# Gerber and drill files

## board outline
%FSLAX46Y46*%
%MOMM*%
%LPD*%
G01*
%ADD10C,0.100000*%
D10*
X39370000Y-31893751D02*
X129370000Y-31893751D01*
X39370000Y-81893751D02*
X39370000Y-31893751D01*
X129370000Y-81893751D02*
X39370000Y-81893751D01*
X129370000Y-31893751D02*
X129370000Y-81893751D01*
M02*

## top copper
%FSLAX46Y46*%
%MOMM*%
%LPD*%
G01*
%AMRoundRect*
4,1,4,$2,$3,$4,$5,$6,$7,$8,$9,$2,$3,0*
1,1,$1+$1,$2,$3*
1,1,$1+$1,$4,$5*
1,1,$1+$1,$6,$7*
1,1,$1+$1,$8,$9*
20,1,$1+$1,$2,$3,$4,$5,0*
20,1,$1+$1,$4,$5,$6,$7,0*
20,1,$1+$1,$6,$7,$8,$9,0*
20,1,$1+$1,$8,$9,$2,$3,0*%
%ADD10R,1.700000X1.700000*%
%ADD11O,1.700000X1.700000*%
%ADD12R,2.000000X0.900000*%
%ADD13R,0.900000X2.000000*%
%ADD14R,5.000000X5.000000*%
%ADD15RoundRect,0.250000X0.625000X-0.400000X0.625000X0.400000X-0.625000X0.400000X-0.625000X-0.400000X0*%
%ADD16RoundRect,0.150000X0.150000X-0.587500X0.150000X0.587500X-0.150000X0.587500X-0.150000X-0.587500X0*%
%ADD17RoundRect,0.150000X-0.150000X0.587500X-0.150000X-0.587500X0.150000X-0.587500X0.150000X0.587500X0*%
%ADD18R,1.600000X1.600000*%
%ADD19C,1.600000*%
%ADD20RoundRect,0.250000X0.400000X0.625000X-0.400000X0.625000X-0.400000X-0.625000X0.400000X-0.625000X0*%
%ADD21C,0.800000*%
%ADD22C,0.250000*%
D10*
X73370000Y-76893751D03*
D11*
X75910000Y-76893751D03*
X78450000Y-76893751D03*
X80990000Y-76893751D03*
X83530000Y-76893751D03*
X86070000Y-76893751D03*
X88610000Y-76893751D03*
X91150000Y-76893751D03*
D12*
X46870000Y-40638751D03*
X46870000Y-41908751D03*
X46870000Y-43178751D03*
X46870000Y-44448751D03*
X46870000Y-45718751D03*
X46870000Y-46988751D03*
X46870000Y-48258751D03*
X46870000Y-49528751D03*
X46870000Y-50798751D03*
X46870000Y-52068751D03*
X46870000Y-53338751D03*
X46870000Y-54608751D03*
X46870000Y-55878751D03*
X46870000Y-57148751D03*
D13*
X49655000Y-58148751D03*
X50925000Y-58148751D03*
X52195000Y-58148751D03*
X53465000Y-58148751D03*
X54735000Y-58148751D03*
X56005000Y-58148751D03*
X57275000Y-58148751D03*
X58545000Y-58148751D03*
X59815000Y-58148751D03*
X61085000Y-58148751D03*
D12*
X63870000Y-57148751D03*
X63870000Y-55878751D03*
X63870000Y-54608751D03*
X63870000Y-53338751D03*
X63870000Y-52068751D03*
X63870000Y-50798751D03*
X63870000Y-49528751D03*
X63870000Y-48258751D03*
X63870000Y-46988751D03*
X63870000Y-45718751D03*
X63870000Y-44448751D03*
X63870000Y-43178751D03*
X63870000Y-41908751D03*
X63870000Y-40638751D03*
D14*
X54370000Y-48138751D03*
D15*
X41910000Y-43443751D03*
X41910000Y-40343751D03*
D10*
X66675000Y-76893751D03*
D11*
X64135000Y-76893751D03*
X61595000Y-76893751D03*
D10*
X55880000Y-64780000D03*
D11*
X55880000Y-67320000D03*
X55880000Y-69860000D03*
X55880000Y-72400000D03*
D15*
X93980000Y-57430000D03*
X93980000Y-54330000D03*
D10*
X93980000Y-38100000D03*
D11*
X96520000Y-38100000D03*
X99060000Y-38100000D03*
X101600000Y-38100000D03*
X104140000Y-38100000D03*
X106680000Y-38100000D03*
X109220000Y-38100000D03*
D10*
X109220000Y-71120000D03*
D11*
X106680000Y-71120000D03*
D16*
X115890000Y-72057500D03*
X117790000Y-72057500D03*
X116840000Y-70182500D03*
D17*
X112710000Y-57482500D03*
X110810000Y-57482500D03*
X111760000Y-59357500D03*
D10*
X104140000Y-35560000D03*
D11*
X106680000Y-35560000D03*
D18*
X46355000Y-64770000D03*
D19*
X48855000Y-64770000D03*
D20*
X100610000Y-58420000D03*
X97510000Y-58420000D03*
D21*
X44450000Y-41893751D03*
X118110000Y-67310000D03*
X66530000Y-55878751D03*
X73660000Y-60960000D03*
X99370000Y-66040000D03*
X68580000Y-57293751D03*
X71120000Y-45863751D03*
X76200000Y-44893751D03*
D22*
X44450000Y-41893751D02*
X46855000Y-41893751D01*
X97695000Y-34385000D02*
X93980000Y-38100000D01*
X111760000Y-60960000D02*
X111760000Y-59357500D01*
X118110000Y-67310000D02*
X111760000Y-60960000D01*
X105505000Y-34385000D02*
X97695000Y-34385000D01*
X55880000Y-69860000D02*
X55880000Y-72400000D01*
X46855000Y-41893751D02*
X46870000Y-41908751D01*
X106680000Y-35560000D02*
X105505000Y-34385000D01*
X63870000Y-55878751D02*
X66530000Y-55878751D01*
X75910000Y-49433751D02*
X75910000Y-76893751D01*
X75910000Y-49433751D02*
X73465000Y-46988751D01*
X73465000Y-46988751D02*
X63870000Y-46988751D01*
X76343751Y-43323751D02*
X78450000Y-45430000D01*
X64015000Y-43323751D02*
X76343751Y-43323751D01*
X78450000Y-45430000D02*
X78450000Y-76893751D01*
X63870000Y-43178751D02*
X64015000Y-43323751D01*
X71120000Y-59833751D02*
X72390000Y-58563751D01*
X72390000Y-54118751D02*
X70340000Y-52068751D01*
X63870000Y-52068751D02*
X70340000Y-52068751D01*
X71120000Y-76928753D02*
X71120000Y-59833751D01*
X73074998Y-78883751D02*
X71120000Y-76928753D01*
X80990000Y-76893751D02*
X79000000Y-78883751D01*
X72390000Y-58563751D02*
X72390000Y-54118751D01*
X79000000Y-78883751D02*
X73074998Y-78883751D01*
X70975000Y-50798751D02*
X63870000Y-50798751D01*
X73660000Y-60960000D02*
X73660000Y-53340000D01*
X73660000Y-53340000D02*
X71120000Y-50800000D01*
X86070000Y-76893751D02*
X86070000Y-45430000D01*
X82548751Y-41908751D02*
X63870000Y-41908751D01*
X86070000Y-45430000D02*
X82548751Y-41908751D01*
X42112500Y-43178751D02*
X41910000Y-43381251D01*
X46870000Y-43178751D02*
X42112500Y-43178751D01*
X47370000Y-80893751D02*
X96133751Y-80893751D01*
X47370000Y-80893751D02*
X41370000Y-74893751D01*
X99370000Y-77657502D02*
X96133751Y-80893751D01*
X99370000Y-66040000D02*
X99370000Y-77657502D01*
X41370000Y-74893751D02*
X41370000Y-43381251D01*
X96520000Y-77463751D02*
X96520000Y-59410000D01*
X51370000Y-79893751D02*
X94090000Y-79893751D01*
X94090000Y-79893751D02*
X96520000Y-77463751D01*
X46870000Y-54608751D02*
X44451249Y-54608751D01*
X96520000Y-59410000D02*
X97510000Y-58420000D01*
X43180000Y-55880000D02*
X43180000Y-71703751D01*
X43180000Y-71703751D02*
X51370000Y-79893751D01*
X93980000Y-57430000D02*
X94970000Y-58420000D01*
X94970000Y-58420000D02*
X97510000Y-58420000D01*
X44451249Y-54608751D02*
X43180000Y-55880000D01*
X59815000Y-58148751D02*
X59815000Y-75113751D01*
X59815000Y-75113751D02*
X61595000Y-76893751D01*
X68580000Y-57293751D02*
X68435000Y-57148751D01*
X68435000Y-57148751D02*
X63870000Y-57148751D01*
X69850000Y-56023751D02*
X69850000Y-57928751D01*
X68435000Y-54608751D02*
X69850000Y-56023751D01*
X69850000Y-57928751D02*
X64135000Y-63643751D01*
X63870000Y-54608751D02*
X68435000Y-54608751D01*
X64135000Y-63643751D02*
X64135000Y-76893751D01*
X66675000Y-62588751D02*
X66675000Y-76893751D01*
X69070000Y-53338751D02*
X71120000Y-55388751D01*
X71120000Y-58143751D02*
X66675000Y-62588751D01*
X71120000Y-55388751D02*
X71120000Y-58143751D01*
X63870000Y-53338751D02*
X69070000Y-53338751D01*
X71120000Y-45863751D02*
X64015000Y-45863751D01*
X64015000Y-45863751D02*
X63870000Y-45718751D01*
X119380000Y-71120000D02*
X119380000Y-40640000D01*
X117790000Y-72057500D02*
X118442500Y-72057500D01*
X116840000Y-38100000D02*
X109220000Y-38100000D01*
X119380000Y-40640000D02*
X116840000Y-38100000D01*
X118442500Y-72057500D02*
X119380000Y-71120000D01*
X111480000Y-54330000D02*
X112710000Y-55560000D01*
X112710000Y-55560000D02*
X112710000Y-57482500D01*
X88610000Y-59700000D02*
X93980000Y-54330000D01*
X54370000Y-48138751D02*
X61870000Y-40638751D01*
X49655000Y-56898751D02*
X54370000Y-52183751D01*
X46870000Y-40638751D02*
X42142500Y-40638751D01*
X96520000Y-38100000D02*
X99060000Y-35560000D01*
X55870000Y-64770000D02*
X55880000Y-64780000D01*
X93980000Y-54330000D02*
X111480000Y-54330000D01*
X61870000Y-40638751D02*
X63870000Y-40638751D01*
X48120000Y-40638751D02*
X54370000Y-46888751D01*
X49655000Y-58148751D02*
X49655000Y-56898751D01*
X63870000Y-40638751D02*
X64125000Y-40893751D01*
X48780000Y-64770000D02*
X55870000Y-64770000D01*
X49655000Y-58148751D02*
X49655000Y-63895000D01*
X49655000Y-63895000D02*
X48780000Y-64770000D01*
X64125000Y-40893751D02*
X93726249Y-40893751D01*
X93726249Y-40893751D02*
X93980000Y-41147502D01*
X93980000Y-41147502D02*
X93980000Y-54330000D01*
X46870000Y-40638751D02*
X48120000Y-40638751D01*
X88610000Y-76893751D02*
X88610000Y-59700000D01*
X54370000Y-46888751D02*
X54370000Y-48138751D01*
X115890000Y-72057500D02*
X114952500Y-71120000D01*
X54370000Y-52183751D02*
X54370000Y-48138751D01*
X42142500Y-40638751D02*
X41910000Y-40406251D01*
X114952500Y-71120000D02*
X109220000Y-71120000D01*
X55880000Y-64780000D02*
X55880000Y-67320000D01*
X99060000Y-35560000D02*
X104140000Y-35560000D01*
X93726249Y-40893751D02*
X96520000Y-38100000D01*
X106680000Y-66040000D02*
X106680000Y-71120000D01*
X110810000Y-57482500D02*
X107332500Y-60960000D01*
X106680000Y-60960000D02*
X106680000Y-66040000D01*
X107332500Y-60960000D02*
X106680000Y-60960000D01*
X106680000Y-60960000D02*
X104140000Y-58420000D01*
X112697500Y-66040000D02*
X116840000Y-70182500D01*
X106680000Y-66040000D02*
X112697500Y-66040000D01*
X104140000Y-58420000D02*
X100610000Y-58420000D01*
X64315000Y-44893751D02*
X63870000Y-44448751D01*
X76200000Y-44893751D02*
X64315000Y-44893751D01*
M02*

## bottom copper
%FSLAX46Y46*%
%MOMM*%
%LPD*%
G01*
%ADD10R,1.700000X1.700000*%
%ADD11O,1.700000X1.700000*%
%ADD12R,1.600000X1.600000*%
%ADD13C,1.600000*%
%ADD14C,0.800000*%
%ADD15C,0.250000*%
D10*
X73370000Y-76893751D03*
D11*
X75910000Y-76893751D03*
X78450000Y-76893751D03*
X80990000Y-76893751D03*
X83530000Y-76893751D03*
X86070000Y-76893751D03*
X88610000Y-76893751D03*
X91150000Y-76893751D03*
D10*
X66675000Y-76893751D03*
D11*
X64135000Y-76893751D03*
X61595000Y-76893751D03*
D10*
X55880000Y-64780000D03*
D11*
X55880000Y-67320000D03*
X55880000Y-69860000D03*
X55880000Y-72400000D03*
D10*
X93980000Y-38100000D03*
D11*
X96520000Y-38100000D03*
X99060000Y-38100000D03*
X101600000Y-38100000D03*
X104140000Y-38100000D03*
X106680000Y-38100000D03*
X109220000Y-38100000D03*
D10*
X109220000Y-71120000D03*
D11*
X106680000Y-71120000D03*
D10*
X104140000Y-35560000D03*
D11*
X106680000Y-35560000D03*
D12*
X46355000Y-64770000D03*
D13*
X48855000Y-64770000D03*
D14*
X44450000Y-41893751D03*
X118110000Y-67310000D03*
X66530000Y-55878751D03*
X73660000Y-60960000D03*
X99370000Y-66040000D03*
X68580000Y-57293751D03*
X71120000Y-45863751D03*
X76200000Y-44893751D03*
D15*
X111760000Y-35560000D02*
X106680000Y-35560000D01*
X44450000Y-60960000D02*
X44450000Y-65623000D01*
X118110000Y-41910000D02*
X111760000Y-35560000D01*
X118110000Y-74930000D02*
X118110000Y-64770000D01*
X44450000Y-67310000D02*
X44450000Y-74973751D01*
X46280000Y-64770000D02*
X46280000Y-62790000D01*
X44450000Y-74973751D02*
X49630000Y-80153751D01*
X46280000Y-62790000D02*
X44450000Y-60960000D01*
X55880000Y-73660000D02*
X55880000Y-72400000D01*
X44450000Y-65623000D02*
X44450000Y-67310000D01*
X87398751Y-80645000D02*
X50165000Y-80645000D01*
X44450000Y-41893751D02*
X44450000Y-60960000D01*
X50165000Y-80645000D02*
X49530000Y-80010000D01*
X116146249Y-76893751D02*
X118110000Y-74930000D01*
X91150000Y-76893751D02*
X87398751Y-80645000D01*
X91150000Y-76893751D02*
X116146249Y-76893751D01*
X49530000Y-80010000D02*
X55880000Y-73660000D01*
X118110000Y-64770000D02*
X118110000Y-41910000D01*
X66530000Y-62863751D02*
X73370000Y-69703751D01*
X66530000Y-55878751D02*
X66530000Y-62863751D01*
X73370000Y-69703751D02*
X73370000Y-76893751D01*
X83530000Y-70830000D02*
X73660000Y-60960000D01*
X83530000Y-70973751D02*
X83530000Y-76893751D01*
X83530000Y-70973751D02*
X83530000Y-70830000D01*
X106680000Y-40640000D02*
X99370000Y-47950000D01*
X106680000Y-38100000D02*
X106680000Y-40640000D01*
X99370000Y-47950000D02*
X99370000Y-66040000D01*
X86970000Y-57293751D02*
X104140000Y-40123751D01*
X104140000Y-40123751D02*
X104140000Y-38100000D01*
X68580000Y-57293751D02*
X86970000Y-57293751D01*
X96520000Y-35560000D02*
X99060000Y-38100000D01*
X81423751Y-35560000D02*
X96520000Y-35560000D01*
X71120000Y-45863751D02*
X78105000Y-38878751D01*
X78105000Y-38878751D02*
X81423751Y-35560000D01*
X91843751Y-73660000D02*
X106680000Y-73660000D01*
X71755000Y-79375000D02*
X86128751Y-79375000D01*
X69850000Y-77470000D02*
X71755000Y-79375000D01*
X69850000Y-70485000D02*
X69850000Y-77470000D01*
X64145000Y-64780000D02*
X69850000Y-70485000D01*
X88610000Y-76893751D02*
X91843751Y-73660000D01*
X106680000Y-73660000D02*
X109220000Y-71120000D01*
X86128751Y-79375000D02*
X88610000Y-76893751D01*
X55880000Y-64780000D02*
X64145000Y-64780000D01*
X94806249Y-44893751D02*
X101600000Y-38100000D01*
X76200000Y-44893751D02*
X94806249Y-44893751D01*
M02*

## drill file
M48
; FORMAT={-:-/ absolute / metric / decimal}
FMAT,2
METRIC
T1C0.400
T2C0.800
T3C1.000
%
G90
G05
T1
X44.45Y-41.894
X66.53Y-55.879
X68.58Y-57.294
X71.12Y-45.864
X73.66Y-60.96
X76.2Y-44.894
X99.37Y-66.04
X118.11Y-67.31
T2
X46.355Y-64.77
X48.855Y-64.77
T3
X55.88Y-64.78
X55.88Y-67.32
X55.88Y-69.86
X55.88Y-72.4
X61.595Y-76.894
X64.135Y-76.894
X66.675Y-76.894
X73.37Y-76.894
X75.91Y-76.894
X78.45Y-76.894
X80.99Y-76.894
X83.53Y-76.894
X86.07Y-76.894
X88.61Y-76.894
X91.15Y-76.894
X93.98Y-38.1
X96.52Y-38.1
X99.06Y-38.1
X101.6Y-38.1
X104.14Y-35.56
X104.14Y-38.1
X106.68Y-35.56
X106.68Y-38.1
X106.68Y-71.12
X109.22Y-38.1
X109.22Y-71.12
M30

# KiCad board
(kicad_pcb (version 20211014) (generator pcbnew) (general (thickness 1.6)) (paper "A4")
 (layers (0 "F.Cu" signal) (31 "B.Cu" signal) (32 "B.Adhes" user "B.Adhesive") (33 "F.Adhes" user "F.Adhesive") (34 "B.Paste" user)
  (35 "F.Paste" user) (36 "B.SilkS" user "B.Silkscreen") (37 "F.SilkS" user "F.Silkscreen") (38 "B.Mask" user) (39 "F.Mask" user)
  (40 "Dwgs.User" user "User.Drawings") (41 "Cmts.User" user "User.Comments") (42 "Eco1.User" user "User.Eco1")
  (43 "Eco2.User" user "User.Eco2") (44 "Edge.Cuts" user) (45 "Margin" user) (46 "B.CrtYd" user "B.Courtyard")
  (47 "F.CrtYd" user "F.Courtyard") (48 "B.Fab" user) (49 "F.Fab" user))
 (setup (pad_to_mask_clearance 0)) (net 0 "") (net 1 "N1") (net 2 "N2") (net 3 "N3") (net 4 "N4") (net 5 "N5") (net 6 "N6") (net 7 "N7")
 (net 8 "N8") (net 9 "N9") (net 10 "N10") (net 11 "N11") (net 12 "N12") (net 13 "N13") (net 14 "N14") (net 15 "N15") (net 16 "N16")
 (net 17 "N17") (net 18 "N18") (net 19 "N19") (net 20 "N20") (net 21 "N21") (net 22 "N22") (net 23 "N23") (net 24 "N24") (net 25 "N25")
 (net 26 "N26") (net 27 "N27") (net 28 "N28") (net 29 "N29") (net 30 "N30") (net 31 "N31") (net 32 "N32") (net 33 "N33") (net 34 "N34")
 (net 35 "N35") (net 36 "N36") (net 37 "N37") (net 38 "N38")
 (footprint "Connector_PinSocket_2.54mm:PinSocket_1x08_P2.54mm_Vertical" (layer "F.Cu") (at 73.37 76.893751 90)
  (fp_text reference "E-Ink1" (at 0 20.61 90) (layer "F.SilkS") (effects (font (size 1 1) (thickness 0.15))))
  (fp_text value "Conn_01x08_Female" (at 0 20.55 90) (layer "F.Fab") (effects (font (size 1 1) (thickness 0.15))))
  (pad "1" thru_hole rect locked (at 0 0 90) (size 1.7 1.7) (drill 1) (layers *.Cu *.Mask) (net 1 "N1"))
  (pad "2" thru_hole oval locked (at 0 2.54 90) (size 1.7 1.7) (drill 1) (layers *.Cu *.Mask) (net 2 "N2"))
  (pad "3" thru_hole oval locked (at 0 5.08 90) (size 1.7 1.7) (drill 1) (layers *.Cu *.Mask) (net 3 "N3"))
  (pad "4" thru_hole oval locked (at 0 7.62 90) (size 1.7 1.7) (drill 1) (layers *.Cu *.Mask) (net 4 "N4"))
  (pad "5" thru_hole oval locked (at 0 10.16 90) (size 1.7 1.7) (drill 1) (layers *.Cu *.Mask) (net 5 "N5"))
  (pad "6" thru_hole oval locked (at 0 12.7 90) (size 1.7 1.7) (drill 1) (layers *.Cu *.Mask) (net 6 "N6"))
  (pad "7" thru_hole oval locked (at 0 15.24 90) (size 1.7 1.7) (drill 1) (layers *.Cu *.Mask) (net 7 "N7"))
  (pad "8" thru_hole oval locked (at 0 17.78 90) (size 1.7 1.7) (drill 1) (layers *.Cu *.Mask) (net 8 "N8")))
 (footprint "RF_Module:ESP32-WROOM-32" (layer "F.Cu") (at 55.37 48.893751)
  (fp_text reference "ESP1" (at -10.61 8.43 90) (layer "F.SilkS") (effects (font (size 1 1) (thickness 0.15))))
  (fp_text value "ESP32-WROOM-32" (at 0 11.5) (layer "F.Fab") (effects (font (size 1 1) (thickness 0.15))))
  (pad "1" smd rect locked (at -8.5 -8.255) (size 2 0.9) (layers "F.Cu" "F.Paste" "F.Mask") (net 7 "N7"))
  (pad "2" smd rect locked (at -8.5 -6.985) (size 2 0.9) (layers "F.Cu" "F.Paste" "F.Mask") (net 8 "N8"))
  (pad "3" smd rect locked (at -8.5 -5.715) (size 2 0.9) (layers "F.Cu" "F.Paste" "F.Mask") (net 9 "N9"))
  (pad "4" smd rect locked (at -8.5 -4.445) (size 2 0.9) (layers "F.Cu" "F.Paste" "F.Mask") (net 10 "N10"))
  (pad "5" smd rect locked (at -8.5 -3.175) (size 2 0.9) (layers "F.Cu" "F.Paste" "F.Mask") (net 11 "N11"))
  (pad "6" smd rect locked (at -8.5 -1.905) (size 2 0.9) (layers "F.Cu" "F.Paste" "F.Mask") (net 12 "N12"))
  (pad "7" smd rect locked (at -8.5 -0.635) (size 2 0.9) (layers "F.Cu" "F.Paste" "F.Mask") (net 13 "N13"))
  (pad "8" smd rect locked (at -8.5 0.635) (size 2 0.9) (layers "F.Cu" "F.Paste" "F.Mask") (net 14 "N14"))
  (pad "9" smd rect locked (at -8.5 1.905) (size 2 0.9) (layers "F.Cu" "F.Paste" "F.Mask") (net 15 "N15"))
  (pad "10" smd rect locked (at -8.5 3.175) (size 2 0.9) (layers "F.Cu" "F.Paste" "F.Mask") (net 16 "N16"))
  (pad "11" smd rect locked (at -8.5 4.445) (size 2 0.9) (layers "F.Cu" "F.Paste" "F.Mask") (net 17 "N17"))
  (pad "12" smd rect locked (at -8.5 5.715) (size 2 0.9) (layers "F.Cu" "F.Paste" "F.Mask") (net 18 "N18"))
  (pad "13" smd rect locked (at -8.5 6.985) (size 2 0.9) (layers "F.Cu" "F.Paste" "F.Mask") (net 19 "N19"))
  (pad "14" smd rect locked (at -8.5 8.255) (size 2 0.9) (layers "F.Cu" "F.Paste" "F.Mask") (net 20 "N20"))
  (pad "15" smd rect locked (at -5.715 9.255 90) (size 2 0.9) (layers "F.Cu" "F.Paste" "F.Mask") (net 7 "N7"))
  (pad "16" smd rect locked (at -4.445 9.255 90) (size 2 0.9) (layers "F.Cu" "F.Paste" "F.Mask") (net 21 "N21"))
  (pad "17" smd rect locked (at -3.175 9.255 90) (size 2 0.9) (layers "F.Cu" "F.Paste" "F.Mask") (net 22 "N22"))
  (pad "18" smd rect locked (at -1.905 9.255 90) (size 2 0.9) (layers "F.Cu" "F.Paste" "F.Mask") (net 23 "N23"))
  (pad "19" smd rect locked (at -0.635 9.255 90) (size 2 0.9) (layers "F.Cu" "F.Paste" "F.Mask") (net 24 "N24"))
  (pad "20" smd rect locked (at 0.635 9.255 90) (size 2 0.9) (layers "F.Cu" "F.Paste" "F.Mask") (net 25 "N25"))
  (pad "21" smd rect locked (at 1.905 9.255 90) (size 2 0.9) (layers "F.Cu" "F.Paste" "F.Mask") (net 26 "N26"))
  (pad "22" smd rect locked (at 3.175 9.255 90) (size 2 0.9) (layers "F.Cu" "F.Paste" "F.Mask") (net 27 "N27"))
  (pad "23" smd rect locked (at 4.445 9.255 90) (size 2 0.9) (layers "F.Cu" "F.Paste" "F.Mask") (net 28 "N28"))
  (pad "24" smd rect locked (at 5.715 9.255 90) (size 2 0.9) (layers "F.Cu" "F.Paste" "F.Mask") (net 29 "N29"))
  (pad "25" smd rect locked (at 8.5 8.255) (size 2 0.9) (layers "F.Cu" "F.Paste" "F.Mask") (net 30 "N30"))
  (pad "26" smd rect locked (at 8.5 6.985) (size 2 0.9) (layers "F.Cu" "F.Paste" "F.Mask") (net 1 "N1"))
  (pad "27" smd rect locked (at 8.5 5.715) (size 2 0.9) (layers "F.Cu" "F.Paste" "F.Mask") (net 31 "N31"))
  (pad "28" smd rect locked (at 8.5 4.445) (size 2 0.9) (layers "F.Cu" "F.Paste" "F.Mask") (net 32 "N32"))
  (pad "29" smd rect locked (at 8.5 3.175) (size 2 0.9) (layers "F.Cu" "F.Paste" "F.Mask") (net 4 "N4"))
  (pad "30" smd rect locked (at 8.5 1.905) (size 2 0.9) (layers "F.Cu" "F.Paste" "F.Mask") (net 5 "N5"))
  (pad "31" smd rect locked (at 8.5 0.635) (size 2 0.9) (layers "F.Cu" "F.Paste" "F.Mask") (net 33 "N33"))
  (pad "32" smd rect locked (at 8.5 -0.635) (size 2 0.9) (layers "F.Cu" "F.Paste" "F.Mask") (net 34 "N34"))
  (pad "33" smd rect locked (at 8.5 -1.905) (size 2 0.9) (layers "F.Cu" "F.Paste" "F.Mask") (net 2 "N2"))
  (pad "34" smd rect locked (at 8.5 -3.175) (size 2 0.9) (layers "F.Cu" "F.Paste" "F.Mask") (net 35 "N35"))
  (pad "35" smd rect locked (at 8.5 -4.445) (size 2 0.9) (layers "F.Cu" "F.Paste" "F.Mask") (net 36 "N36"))
  (pad "36" smd rect locked (at 8.5 -5.715) (size 2 0.9) (layers "F.Cu" "F.Paste" "F.Mask") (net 3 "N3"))
  (pad "37" smd rect locked (at 8.5 -6.985) (size 2 0.9) (layers "F.Cu" "F.Paste" "F.Mask") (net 6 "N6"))
  (pad "38" smd rect locked (at 8.5 -8.255) (size 2 0.9) (layers "F.Cu" "F.Paste" "F.Mask") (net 7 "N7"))
  (pad "39" smd rect locked (at -1 -0.755) (size 5 5) (layers "F.Cu" "F.Paste" "F.Mask") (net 7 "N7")))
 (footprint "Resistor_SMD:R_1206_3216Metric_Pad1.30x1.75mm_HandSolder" (layer "F.Cu") (at 41.91 41.893751 90)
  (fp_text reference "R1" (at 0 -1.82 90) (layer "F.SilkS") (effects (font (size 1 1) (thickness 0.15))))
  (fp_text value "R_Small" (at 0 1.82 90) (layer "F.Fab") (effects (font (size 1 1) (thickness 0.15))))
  (pad "1" smd roundrect (at -1.55 0 90) (size 1.3 1.75) (layers "F.Cu" "F.Paste" "F.Mask") (roundrect_rratio 0.192308) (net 9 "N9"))
  (pad "2" smd roundrect (at 1.55 0 90) (size 1.3 1.75) (layers "F.Cu" "F.Paste" "F.Mask") (roundrect_rratio 0.192308) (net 7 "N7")))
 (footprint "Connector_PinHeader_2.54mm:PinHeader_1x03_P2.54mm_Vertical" (layer "F.Cu") (at 66.675 76.893751 -90)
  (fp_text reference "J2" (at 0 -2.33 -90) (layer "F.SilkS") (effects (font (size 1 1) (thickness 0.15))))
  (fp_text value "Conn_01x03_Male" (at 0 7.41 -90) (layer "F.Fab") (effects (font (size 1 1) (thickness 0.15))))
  (pad "1" thru_hole rect (at 0 0 270) (size 1.7 1.7) (drill 1) (layers *.Cu *.Mask) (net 32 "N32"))
  (pad "2" thru_hole oval (at 0 2.54 270) (size 1.7 1.7) (drill 1) (layers *.Cu *.Mask) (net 31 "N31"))
  (pad "3" thru_hole oval (at 0 5.08 270) (size 1.7 1.7) (drill 1) (layers *.Cu *.Mask) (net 28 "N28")))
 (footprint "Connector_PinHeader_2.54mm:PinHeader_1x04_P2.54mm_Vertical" (layer "F.Cu") (at 55.88 64.78)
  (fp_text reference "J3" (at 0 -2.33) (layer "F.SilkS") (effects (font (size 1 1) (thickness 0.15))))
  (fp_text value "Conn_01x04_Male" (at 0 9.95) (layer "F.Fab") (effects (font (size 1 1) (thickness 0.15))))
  (pad "1" thru_hole rect (at 0 0) (size 1.7 1.7) (drill 1) (layers *.Cu *.Mask) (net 7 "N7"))
  (pad "2" thru_hole oval (at 0 2.54) (size 1.7 1.7) (drill 1) (layers *.Cu *.Mask) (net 7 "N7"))
  (pad "3" thru_hole oval (at 0 5.08) (size 1.7 1.7) (drill 1) (layers *.Cu *.Mask) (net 8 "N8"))
  (pad "4" thru_hole oval (at 0 7.62) (size 1.7 1.7) (drill 1) (layers *.Cu *.Mask) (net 8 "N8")))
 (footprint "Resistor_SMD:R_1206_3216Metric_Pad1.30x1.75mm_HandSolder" (layer "F.Cu") (at 93.98 55.88 90)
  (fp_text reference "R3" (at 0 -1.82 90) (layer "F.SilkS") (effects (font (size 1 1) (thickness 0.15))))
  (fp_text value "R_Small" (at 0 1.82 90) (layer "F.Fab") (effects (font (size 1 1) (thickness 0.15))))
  (pad "1" smd roundrect (at -1.55 0 90) (size 1.3 1.75) (layers "F.Cu" "F.Paste" "F.Mask") (roundrect_rratio 0.192308) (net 18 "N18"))
  (pad "2" smd roundrect (at 1.55 0 90) (size 1.3 1.75) (layers "F.Cu" "F.Paste" "F.Mask") (roundrect_rratio 0.192308) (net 7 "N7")))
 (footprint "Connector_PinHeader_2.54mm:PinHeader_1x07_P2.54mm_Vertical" (layer "F.Cu") (at 93.98 38.1 90)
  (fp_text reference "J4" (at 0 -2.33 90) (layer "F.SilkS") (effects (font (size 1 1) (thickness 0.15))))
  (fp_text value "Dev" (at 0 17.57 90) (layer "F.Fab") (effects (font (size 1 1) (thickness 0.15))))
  (pad "1" thru_hole rect (at 0 0 90) (size 1.7 1.7) (drill 1) (layers *.Cu *.Mask) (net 8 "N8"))
  (pad "2" thru_hole oval (at 0 2.54 90) (size 1.7 1.7) (drill 1) (layers *.Cu *.Mask) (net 7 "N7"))
  (pad "3" thru_hole oval (at 0 5.08 90) (size 1.7 1.7) (drill 1) (layers *.Cu *.Mask) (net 35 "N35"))
  (pad "4" thru_hole oval (at 0 7.62 90) (size 1.7 1.7) (drill 1) (layers *.Cu *.Mask) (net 36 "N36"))
  (pad "5" thru_hole oval (at 0 10.16 90) (size 1.7 1.7) (drill 1) (layers *.Cu *.Mask) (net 30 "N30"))
  (pad "6" thru_hole oval (at 0 12.7 90) (size 1.7 1.7) (drill 1) (layers *.Cu *.Mask) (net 9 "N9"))
  (pad "7" thru_hole oval (at 0 15.24 90) (size 1.7 1.7) (drill 1) (layers *.Cu *.Mask) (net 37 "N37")))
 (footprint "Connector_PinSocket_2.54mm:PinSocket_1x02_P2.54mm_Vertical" (layer "F.Cu") (at 109.22 71.12 -90)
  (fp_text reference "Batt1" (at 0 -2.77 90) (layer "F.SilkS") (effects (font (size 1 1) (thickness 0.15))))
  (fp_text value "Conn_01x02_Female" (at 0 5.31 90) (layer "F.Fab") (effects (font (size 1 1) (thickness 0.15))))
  (pad "1" thru_hole rect (at 0 0 270) (size 1.7 1.7) (drill 1) (layers *.Cu *.Mask) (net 7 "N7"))
  (pad "2" thru_hole oval (at 0 2.54 270) (size 1.7 1.7) (drill 1) (layers *.Cu *.Mask) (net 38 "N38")))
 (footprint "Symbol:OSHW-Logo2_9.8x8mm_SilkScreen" (layer "F.Cu") (at 122.555 38.735)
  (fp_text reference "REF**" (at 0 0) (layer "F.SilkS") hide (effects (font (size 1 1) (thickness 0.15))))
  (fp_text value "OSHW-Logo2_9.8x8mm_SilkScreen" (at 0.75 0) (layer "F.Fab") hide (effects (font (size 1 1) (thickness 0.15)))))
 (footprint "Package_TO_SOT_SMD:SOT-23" (layer "F.Cu") (at 116.84 71.12 90)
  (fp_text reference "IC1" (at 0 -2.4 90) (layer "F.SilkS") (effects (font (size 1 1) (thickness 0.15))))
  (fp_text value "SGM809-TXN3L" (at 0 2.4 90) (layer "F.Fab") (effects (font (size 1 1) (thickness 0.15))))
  (pad "1" smd roundrect (at -0.9375 -0.95 90) (size 1.475 0.6) (layers "F.Cu" "F.Paste" "F.Mask") (roundrect_rratio 0.25) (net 7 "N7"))
  (pad "2" smd roundrect (at -0.9375 0.95 90) (size 1.475 0.6) (layers "F.Cu" "F.Paste" "F.Mask") (roundrect_rratio 0.25) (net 37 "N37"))
  (pad "3" smd roundrect (at 0.9375 0 90) (size 1.475 0.6) (layers "F.Cu" "F.Paste" "F.Mask") (roundrect_rratio 0.25) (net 38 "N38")))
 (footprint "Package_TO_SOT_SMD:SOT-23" (layer "F.Cu") (at 111.76 58.42 -90)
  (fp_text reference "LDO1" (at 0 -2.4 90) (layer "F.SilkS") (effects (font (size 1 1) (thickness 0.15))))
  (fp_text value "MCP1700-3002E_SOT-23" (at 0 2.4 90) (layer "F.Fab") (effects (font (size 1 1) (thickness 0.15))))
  (pad "1" smd roundrect (at -0.9375 -0.95 270) (size 1.475 0.6) (layers "F.Cu" "F.Paste" "F.Mask") (roundrect_rratio 0.25) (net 7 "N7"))
  (pad "2" smd roundrect (at -0.9375 0.95 270) (size 1.475 0.6) (layers "F.Cu" "F.Paste" "F.Mask") (roundrect_rratio 0.25) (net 38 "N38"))
  (pad "3" smd roundrect (at 0.9375 0 270) (size 1.475 0.6) (layers "F.Cu" "F.Paste" "F.Mask") (roundrect_rratio 0.25) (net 8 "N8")))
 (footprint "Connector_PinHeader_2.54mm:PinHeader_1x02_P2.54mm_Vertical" (layer "F.Cu") (at 104.14 35.56 90)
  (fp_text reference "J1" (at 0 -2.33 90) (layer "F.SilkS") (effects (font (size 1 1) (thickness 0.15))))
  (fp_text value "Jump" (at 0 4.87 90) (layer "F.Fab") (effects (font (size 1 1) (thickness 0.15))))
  (pad "1" thru_hole rect (at 0 0 90) (size 1.7 1.7) (drill 1) (layers *.Cu *.Mask) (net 7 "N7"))
  (pad "2" thru_hole oval (at 0 2.54 90) (size 1.7 1.7) (drill 1) (layers *.Cu *.Mask) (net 8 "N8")))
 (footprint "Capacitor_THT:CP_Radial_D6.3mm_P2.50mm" (layer "F.Cu") (at 46.355 64.77)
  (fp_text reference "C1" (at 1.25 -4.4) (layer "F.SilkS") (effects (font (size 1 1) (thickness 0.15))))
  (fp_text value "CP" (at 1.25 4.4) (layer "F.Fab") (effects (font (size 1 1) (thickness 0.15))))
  (pad "1" thru_hole rect (at 0 0) (size 1.6 1.6) (drill 0.8) (layers *.Cu *.Mask) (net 8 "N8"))
  (pad "2" thru_hole circle (at 2.5 0) (size 1.6 1.6) (drill 0.8) (layers *.Cu *.Mask) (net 7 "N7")))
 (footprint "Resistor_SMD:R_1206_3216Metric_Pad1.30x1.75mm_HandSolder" (layer "F.Cu") (at 99.06 58.42 180)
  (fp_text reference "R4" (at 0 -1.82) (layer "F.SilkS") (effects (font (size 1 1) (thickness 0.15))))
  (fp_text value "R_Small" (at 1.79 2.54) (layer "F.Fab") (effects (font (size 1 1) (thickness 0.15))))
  (pad "1" smd roundrect (at -1.55 0 180) (size 1.3 1.75) (layers "F.Cu" "F.Paste" "F.Mask") (roundrect_rratio 0.192308) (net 38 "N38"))
  (pad "2" smd roundrect (at 1.55 0 180) (size 1.3 1.75) (layers "F.Cu" "F.Paste" "F.Mask") (roundrect_rratio 0.192308) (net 18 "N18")))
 (gr_line (start 39.37 31.893751) (end 129.37 31.893751) (layer "Edge.Cuts") (width 0.1))
 (gr_line (start 39.37 81.893751) (end 39.37 31.893751) (layer "Edge.Cuts") (width 0.1))
 (gr_line (start 129.37 81.893751) (end 39.37 81.893751) (layer "Edge.Cuts") (width 0.1))
 (gr_line (start 129.37 31.893751) (end 129.37 81.893751) (layer "Edge.Cuts") (width 0.1))
 (segment (start 44.45 41.893751) (end 46.855 41.893751) (width 0.25) (layer "F.Cu") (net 8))
 (segment (start 97.695 34.385) (end 93.98 38.1) (width 0.25) (layer "F.Cu") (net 8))
 (segment (start 111.76 60.96) (end 111.76 59.3575) (width 0.25) (layer "F.Cu") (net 8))
 (segment (start 118.11 67.31) (end 111.76 60.96) (width 0.25) (layer "F.Cu") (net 8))
 (segment (start 105.505 34.385) (end 97.695 34.385) (width 0.25) (layer "F.Cu") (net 8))
 (segment (start 55.88 69.86) (end 55.88 72.4) (width 0.25) (layer "F.Cu") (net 8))
 (segment (start 46.855 41.893751) (end 46.87 41.908751) (width 0.25) (layer "F.Cu") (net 8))
 (segment (start 106.68 35.56) (end 105.505 34.385) (width 0.25) (layer "F.Cu") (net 8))
 (via (at 44.45 41.893751) (size 0.8) (drill 0.4) (layers "F.Cu" "B.Cu") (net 8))
 (via (at 118.11 67.31) (size 0.8) (drill 0.4) (layers "F.Cu" "B.Cu") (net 8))
 (segment (start 111.76 35.56) (end 106.68 35.56) (width 0.25) (layer "B.Cu") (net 8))
 (segment (start 44.45 60.96) (end 44.45 65.623) (width 0.25) (layer "B.Cu") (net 8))
 (segment (start 118.11 41.91) (end 111.76 35.56) (width 0.25) (layer "B.Cu") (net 8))
 (segment (start 118.11 74.93) (end 118.11 64.77) (width 0.25) (layer "B.Cu") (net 8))
 (segment (start 44.45 67.31) (end 44.45 74.973751) (width 0.25) (layer "B.Cu") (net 8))
 (segment (start 46.28 64.77) (end 46.28 62.79) (width 0.25) (layer "B.Cu") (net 8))
 (segment (start 44.45 74.973751) (end 49.63 80.153751) (width 0.25) (layer "B.Cu") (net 8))
 (segment (start 46.28 62.79) (end 44.45 60.96) (width 0.25) (layer "B.Cu") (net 8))
 (segment (start 55.88 73.66) (end 55.88 72.4) (width 0.25) (layer "B.Cu") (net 8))
 (segment (start 44.45 65.623) (end 44.45 67.31) (width 0.25) (layer "B.Cu") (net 8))
 (segment (start 87.398751 80.645) (end 50.165 80.645) (width 0.25) (layer "B.Cu") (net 8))
 (segment (start 44.45 41.893751) (end 44.45 60.96) (width 0.25) (layer "B.Cu") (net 8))
 (segment (start 50.165 80.645) (end 49.53 80.01) (width 0.25) (layer "B.Cu") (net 8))
 (segment (start 116.146249 76.893751) (end 118.11 74.93) (width 0.25) (layer "B.Cu") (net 8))
 (segment (start 91.15 76.893751) (end 87.398751 80.645) (width 0.25) (layer "B.Cu") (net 8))
 (segment (start 91.15 76.893751) (end 116.146249 76.893751) (width 0.25) (layer "B.Cu") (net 8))
 (segment (start 49.53 80.01) (end 55.88 73.66) (width 0.25) (layer "B.Cu") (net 8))
 (segment (start 118.11 64.77) (end 118.11 41.91) (width 0.25) (layer "B.Cu") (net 8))
 (segment (start 63.87 55.878751) (end 66.53 55.878751) (width 0.25) (layer "F.Cu") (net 1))
 (via (at 66.53 55.878751) (size 0.8) (drill 0.4) (layers "F.Cu" "B.Cu") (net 1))
 (segment (start 66.53 62.863751) (end 73.37 69.703751) (width 0.25) (layer "B.Cu") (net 1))
 (segment (start 66.53 55.878751) (end 66.53 62.863751) (width 0.25) (layer "B.Cu") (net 1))
 (segment (start 73.37 69.703751) (end 73.37 76.893751) (width 0.25) (layer "B.Cu") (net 1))
 (segment (start 75.91 49.433751) (end 75.91 76.893751) (width 0.25) (layer "F.Cu") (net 2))
 (segment (start 75.91 49.433751) (end 73.465 46.988751) (width 0.25) (layer "F.Cu") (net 2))
 (segment (start 73.465 46.988751) (end 63.87 46.988751) (width 0.25) (layer "F.Cu") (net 2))
 (segment (start 76.343751 43.323751) (end 78.45 45.43) (width 0.25) (layer "F.Cu") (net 3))
 (segment (start 64.015 43.323751) (end 76.343751 43.323751) (width 0.25) (layer "F.Cu") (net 3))
 (segment (start 78.45 45.43) (end 78.45 76.893751) (width 0.25) (layer "F.Cu") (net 3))
 (segment (start 63.87 43.178751) (end 64.015 43.323751) (width 0.25) (layer "F.Cu") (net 3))
 (segment (start 71.12 59.833751) (end 72.39 58.563751) (width 0.25) (layer "F.Cu") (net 4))
 (segment (start 72.39 54.118751) (end 70.34 52.068751) (width 0.25) (layer "F.Cu") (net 4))
 (segment (start 63.87 52.068751) (end 70.34 52.068751) (width 0.25) (layer "F.Cu") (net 4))
 (segment (start 71.12 76.928753) (end 71.12 59.833751) (width 0.25) (layer "F.Cu") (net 4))
 (segment (start 73.074998 78.883751) (end 71.12 76.928753) (width 0.25) (layer "F.Cu") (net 4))
 (segment (start 80.99 76.893751) (end 79 78.883751) (width 0.25) (layer "F.Cu") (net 4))
 (segment (start 72.39 58.563751) (end 72.39 54.118751) (width 0.25) (layer "F.Cu") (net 4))
 (segment (start 79 78.883751) (end 73.074998 78.883751) (width 0.25) (layer "F.Cu") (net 4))
 (segment (start 70.975 50.798751) (end 63.87 50.798751) (width 0.25) (layer "F.Cu") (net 5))
 (segment (start 73.66 60.96) (end 73.66 53.34) (width 0.25) (layer "F.Cu") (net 5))
 (segment (start 73.66 53.34) (end 71.12 50.8) (width 0.25) (layer "F.Cu") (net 5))
 (via (at 73.66 60.96) (size 0.8) (drill 0.4) (layers "F.Cu" "B.Cu") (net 5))
 (segment (start 83.53 70.83) (end 73.66 60.96) (width 0.25) (layer "B.Cu") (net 5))
 (segment (start 83.53 70.973751) (end 83.53 76.893751) (width 0.25) (layer "B.Cu") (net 5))
 (segment (start 83.53 70.973751) (end 83.53 70.83) (width 0.25) (layer "B.Cu") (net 5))
 (segment (start 86.07 76.893751) (end 86.07 45.43) (width 0.25) (layer "F.Cu") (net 6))
 (segment (start 82.548751 41.908751) (end 63.87 41.908751) (width 0.25) (layer "F.Cu") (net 6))
 (segment (start 86.07 45.43) (end 82.548751 41.908751) (width 0.25) (layer "F.Cu") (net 6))
 (segment (start 42.1125 43.178751) (end 41.91 43.381251) (width 0.25) (layer "F.Cu") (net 9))
 (segment (start 46.87 43.178751) (end 42.1125 43.178751) (width 0.25) (layer "F.Cu") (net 9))
 (segment (start 47.37 80.893751) (end 96.133751 80.893751) (width 0.25) (layer "F.Cu") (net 9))
 (segment (start 47.37 80.893751) (end 41.37 74.893751) (width 0.25) (layer "F.Cu") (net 9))
 (segment (start 99.37 77.657502) (end 96.133751 80.893751) (width 0.25) (layer "F.Cu") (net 9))
 (segment (start 99.37 66.04) (end 99.37 77.657502) (width 0.25) (layer "F.Cu") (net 9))
 (segment (start 41.37 74.893751) (end 41.37 43.381251) (width 0.25) (layer "F.Cu") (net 9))
 (via (at 99.37 66.04) (size 0.8) (drill 0.4) (layers "F.Cu" "B.Cu") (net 9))
 (segment (start 106.68 40.64) (end 99.37 47.95) (width 0.25) (layer "B.Cu") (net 9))
 (segment (start 106.68 38.1) (end 106.68 40.64) (width 0.25) (layer "B.Cu") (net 9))
 (segment (start 99.37 47.95) (end 99.37 66.04) (width 0.25) (layer "B.Cu") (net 9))
 (segment (start 96.52 77.463751) (end 96.52 59.41) (width 0.25) (layer "F.Cu") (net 18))
 (segment (start 51.37 79.893751) (end 94.09 79.893751) (width 0.25) (layer "F.Cu") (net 18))
 (segment (start 94.09 79.893751) (end 96.52 77.463751) (width 0.25) (layer "F.Cu") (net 18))
 (segment (start 46.87 54.608751) (end 44.451249 54.608751) (width 0.25) (layer "F.Cu") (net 18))
 (segment (start 96.52 59.41) (end 97.51 58.42) (width 0.25) (layer "F.Cu") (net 18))
 (segment (start 43.18 55.88) (end 43.18 71.703751) (width 0.25) (layer "F.Cu") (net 18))
 (segment (start 43.18 71.703751) (end 51.37 79.893751) (width 0.25) (layer "F.Cu") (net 18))
 (segment (start 93.98 57.43) (end 94.97 58.42) (width 0.25) (layer "F.Cu") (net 18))
 (segment (start 94.97 58.42) (end 97.51 58.42) (width 0.25) (layer "F.Cu") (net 18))
 (segment (start 44.451249 54.608751) (end 43.18 55.88) (width 0.25) (layer "F.Cu") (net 18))
 (segment (start 59.815 58.148751) (end 59.815 75.113751) (width 0.25) (layer "F.Cu") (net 28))
 (segment (start 59.815 75.113751) (end 61.595 76.893751) (width 0.25) (layer "F.Cu") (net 28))
 (segment (start 68.58 57.293751) (end 68.435 57.148751) (width 0.25) (layer "F.Cu") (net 30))
 (segment (start 68.435 57.148751) (end 63.87 57.148751) (width 0.25) (layer "F.Cu") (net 30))
 (via (at 68.58 57.293751) (size 0.8) (drill 0.4) (layers "F.Cu" "B.Cu") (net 30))
 (segment (start 86.97 57.293751) (end 104.14 40.123751) (width 0.25) (layer "B.Cu") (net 30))
 (segment (start 104.14 40.123751) (end 104.14 38.1) (width 0.25) (layer "B.Cu") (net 30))
 (segment (start 68.58 57.293751) (end 86.97 57.293751) (width 0.25) (layer "B.Cu") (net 30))
 (segment (start 69.85 56.023751) (end 69.85 57.928751) (width 0.25) (layer "F.Cu") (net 31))
 (segment (start 68.435 54.608751) (end 69.85 56.023751) (width 0.25) (layer "F.Cu") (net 31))
 (segment (start 69.85 57.928751) (end 64.135 63.643751) (width 0.25) (layer "F.Cu") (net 31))
 (segment (start 63.87 54.608751) (end 68.435 54.608751) (width 0.25) (layer "F.Cu") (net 31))
 (segment (start 64.135 63.643751) (end 64.135 76.893751) (width 0.25) (layer "F.Cu") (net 31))
 (segment (start 66.675 62.588751) (end 66.675 76.893751) (width 0.25) (layer "F.Cu") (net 32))
 (segment (start 69.07 53.338751) (end 71.12 55.388751) (width 0.25) (layer "F.Cu") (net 32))
 (segment (start 71.12 58.143751) (end 66.675 62.588751) (width 0.25) (layer "F.Cu") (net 32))
 (segment (start 71.12 55.388751) (end 71.12 58.143751) (width 0.25) (layer "F.Cu") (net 32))
 (segment (start 63.87 53.338751) (end 69.07 53.338751) (width 0.25) (layer "F.Cu") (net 32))
 (segment (start 71.12 45.863751) (end 64.015 45.863751) (width 0.25) (layer "F.Cu") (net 35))
 (segment (start 64.015 45.863751) (end 63.87 45.718751) (width 0.25) (layer "F.Cu") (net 35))
 (via (at 71.12 45.863751) (size 0.8) (drill 0.4) (layers "F.Cu" "B.Cu") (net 35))
 (segment (start 96.52 35.56) (end 99.06 38.1) (width 0.25) (layer "B.Cu") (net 35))
 (segment (start 81.423751 35.56) (end 96.52 35.56) (width 0.25) (layer "B.Cu") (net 35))
 (segment (start 71.12 45.863751) (end 78.105 38.878751) (width 0.25) (layer "B.Cu") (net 35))
 (segment (start 78.105 38.878751) (end 81.423751 35.56) (width 0.25) (layer "B.Cu") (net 35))
 (segment (start 119.38 71.12) (end 119.38 40.64) (width 0.25) (layer "F.Cu") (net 37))
 (segment (start 117.79 72.0575) (end 118.4425 72.0575) (width 0.25) (layer "F.Cu") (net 37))
 (segment (start 116.84 38.1) (end 109.22 38.1) (width 0.25) (layer "F.Cu") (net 37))
 (segment (start 119.38 40.64) (end 116.84 38.1) (width 0.25) (layer "F.Cu") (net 37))
 (segment (start 118.4425 72.0575) (end 119.38 71.12) (width 0.25) (layer "F.Cu") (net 37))
 (segment (start 111.48 54.33) (end 112.71 55.56) (width 0.25) (layer "F.Cu") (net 7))
 (segment (start 112.71 55.56) (end 112.71 57.4825) (width 0.25) (layer "F.Cu") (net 7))
 (segment (start 88.61 59.7) (end 93.98 54.33) (width 0.25) (layer "F.Cu") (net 7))
 (segment (start 54.37 48.138751) (end 61.87 40.638751) (width 0.25) (layer "F.Cu") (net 7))
 (segment (start 49.655 56.898751) (end 54.37 52.183751) (width 0.25) (layer "F.Cu") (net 7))
 (segment (start 46.87 40.638751) (end 42.1425 40.638751) (width 0.25) (layer "F.Cu") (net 7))
 (segment (start 96.52 38.1) (end 99.06 35.56) (width 0.25) (layer "F.Cu") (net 7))
 (segment (start 55.87 64.77) (end 55.88 64.78) (width 0.25) (layer "F.Cu") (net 7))
 (segment (start 93.98 54.33) (end 111.48 54.33) (width 0.25) (layer "F.Cu") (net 7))
 (segment (start 61.87 40.638751) (end 63.87 40.638751) (width 0.25) (layer "F.Cu") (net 7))
 (segment (start 48.12 40.638751) (end 54.37 46.888751) (width 0.25) (layer "F.Cu") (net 7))
 (segment (start 49.655 58.148751) (end 49.655 56.898751) (width 0.25) (layer "F.Cu") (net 7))
 (segment (start 63.87 40.638751) (end 64.125 40.893751) (width 0.25) (layer "F.Cu") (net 7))
 (segment (start 48.78 64.77) (end 55.87 64.77) (width 0.25) (layer "F.Cu") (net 7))
 (segment (start 49.655 58.148751) (end 49.655 63.895) (width 0.25) (layer "F.Cu") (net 7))
 (segment (start 49.655 63.895) (end 48.78 64.77) (width 0.25) (layer "F.Cu") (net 7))
 (segment (start 64.125 40.893751) (end 93.726249 40.893751) (width 0.25) (layer "F.Cu") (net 7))
 (segment (start 93.726249 40.893751) (end 93.98 41.147502) (width 0.25) (layer "F.Cu") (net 7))
 (segment (start 93.98 41.147502) (end 93.98 54.33) (width 0.25) (layer "F.Cu") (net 7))
 (segment (start 46.87 40.638751) (end 48.12 40.638751) (width 0.25) (layer "F.Cu") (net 7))
 (segment (start 88.61 76.893751) (end 88.61 59.7) (width 0.25) (layer "F.Cu") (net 7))
 (segment (start 54.37 46.888751) (end 54.37 48.138751) (width 0.25) (layer "F.Cu") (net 7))
 (segment (start 115.89 72.0575) (end 114.9525 71.12) (width 0.25) (layer "F.Cu") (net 7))
 (segment (start 54.37 52.183751) (end 54.37 48.138751) (width 0.25) (layer "F.Cu") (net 7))
 (segment (start 42.1425 40.638751) (end 41.91 40.406251) (width 0.25) (layer "F.Cu") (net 7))
 (segment (start 114.9525 71.12) (end 109.22 71.12) (width 0.25) (layer "F.Cu") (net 7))
 (segment (start 55.88 64.78) (end 55.88 67.32) (width 0.25) (layer "F.Cu") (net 7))
 (segment (start 99.06 35.56) (end 104.14 35.56) (width 0.25) (layer "F.Cu") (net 7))
 (segment (start 93.726249 40.893751) (end 96.52 38.1) (width 0.25) (layer "F.Cu") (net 7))
 (segment (start 91.843751 73.66) (end 106.68 73.66) (width 0.25) (layer "B.Cu") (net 7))
 (segment (start 71.755 79.375) (end 86.128751 79.375) (width 0.25) (layer "B.Cu") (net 7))
 (segment (start 69.85 77.47) (end 71.755 79.375) (width 0.25) (layer "B.Cu") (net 7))
 (segment (start 69.85 70.485) (end 69.85 77.47) (width 0.25) (layer "B.Cu") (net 7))
 (segment (start 64.145 64.78) (end 69.85 70.485) (width 0.25) (layer "B.Cu") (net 7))
 (segment (start 88.61 76.893751) (end 91.843751 73.66) (width 0.25) (layer "B.Cu") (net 7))
 (segment (start 106.68 73.66) (end 109.22 71.12) (width 0.25) (layer "B.Cu") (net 7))
 (segment (start 86.128751 79.375) (end 88.61 76.893751) (width 0.25) (layer "B.Cu") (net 7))
 (segment (start 55.88 64.78) (end 64.145 64.78) (width 0.25) (layer "B.Cu") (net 7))
 (segment (start 106.68 66.04) (end 106.68 71.12) (width 0.25) (layer "F.Cu") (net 38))
 (segment (start 110.81 57.4825) (end 107.3325 60.96) (width 0.25) (layer "F.Cu") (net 38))
 (segment (start 106.68 60.96) (end 106.68 66.04) (width 0.25) (layer "F.Cu") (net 38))
 (segment (start 107.3325 60.96) (end 106.68 60.96) (width 0.25) (layer "F.Cu") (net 38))
 (segment (start 106.68 60.96) (end 104.14 58.42) (width 0.25) (layer "F.Cu") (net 38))
 (segment (start 112.6975 66.04) (end 116.84 70.1825) (width 0.25) (layer "F.Cu") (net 38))
 (segment (start 106.68 66.04) (end 112.6975 66.04) (width 0.25) (layer "F.Cu") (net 38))
 (segment (start 104.14 58.42) (end 100.61 58.42) (width 0.25) (layer "F.Cu") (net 38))
 (segment (start 64.315 44.893751) (end 63.87 44.448751) (width 0.25) (layer "F.Cu") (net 36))
 (segment (start 76.2 44.893751) (end 64.315 44.893751) (width 0.25) (layer "F.Cu") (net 36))
 (via (at 76.2 44.893751) (size 0.8) (drill 0.4) (layers "F.Cu" "B.Cu") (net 36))
 (segment (start 94.806249 44.893751) (end 101.6 38.1) (width 0.25) (layer "B.Cu") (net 36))
 (segment (start 76.2 44.893751) (end 94.806249 44.893751) (width 0.25) (layer "B.Cu") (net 36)))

